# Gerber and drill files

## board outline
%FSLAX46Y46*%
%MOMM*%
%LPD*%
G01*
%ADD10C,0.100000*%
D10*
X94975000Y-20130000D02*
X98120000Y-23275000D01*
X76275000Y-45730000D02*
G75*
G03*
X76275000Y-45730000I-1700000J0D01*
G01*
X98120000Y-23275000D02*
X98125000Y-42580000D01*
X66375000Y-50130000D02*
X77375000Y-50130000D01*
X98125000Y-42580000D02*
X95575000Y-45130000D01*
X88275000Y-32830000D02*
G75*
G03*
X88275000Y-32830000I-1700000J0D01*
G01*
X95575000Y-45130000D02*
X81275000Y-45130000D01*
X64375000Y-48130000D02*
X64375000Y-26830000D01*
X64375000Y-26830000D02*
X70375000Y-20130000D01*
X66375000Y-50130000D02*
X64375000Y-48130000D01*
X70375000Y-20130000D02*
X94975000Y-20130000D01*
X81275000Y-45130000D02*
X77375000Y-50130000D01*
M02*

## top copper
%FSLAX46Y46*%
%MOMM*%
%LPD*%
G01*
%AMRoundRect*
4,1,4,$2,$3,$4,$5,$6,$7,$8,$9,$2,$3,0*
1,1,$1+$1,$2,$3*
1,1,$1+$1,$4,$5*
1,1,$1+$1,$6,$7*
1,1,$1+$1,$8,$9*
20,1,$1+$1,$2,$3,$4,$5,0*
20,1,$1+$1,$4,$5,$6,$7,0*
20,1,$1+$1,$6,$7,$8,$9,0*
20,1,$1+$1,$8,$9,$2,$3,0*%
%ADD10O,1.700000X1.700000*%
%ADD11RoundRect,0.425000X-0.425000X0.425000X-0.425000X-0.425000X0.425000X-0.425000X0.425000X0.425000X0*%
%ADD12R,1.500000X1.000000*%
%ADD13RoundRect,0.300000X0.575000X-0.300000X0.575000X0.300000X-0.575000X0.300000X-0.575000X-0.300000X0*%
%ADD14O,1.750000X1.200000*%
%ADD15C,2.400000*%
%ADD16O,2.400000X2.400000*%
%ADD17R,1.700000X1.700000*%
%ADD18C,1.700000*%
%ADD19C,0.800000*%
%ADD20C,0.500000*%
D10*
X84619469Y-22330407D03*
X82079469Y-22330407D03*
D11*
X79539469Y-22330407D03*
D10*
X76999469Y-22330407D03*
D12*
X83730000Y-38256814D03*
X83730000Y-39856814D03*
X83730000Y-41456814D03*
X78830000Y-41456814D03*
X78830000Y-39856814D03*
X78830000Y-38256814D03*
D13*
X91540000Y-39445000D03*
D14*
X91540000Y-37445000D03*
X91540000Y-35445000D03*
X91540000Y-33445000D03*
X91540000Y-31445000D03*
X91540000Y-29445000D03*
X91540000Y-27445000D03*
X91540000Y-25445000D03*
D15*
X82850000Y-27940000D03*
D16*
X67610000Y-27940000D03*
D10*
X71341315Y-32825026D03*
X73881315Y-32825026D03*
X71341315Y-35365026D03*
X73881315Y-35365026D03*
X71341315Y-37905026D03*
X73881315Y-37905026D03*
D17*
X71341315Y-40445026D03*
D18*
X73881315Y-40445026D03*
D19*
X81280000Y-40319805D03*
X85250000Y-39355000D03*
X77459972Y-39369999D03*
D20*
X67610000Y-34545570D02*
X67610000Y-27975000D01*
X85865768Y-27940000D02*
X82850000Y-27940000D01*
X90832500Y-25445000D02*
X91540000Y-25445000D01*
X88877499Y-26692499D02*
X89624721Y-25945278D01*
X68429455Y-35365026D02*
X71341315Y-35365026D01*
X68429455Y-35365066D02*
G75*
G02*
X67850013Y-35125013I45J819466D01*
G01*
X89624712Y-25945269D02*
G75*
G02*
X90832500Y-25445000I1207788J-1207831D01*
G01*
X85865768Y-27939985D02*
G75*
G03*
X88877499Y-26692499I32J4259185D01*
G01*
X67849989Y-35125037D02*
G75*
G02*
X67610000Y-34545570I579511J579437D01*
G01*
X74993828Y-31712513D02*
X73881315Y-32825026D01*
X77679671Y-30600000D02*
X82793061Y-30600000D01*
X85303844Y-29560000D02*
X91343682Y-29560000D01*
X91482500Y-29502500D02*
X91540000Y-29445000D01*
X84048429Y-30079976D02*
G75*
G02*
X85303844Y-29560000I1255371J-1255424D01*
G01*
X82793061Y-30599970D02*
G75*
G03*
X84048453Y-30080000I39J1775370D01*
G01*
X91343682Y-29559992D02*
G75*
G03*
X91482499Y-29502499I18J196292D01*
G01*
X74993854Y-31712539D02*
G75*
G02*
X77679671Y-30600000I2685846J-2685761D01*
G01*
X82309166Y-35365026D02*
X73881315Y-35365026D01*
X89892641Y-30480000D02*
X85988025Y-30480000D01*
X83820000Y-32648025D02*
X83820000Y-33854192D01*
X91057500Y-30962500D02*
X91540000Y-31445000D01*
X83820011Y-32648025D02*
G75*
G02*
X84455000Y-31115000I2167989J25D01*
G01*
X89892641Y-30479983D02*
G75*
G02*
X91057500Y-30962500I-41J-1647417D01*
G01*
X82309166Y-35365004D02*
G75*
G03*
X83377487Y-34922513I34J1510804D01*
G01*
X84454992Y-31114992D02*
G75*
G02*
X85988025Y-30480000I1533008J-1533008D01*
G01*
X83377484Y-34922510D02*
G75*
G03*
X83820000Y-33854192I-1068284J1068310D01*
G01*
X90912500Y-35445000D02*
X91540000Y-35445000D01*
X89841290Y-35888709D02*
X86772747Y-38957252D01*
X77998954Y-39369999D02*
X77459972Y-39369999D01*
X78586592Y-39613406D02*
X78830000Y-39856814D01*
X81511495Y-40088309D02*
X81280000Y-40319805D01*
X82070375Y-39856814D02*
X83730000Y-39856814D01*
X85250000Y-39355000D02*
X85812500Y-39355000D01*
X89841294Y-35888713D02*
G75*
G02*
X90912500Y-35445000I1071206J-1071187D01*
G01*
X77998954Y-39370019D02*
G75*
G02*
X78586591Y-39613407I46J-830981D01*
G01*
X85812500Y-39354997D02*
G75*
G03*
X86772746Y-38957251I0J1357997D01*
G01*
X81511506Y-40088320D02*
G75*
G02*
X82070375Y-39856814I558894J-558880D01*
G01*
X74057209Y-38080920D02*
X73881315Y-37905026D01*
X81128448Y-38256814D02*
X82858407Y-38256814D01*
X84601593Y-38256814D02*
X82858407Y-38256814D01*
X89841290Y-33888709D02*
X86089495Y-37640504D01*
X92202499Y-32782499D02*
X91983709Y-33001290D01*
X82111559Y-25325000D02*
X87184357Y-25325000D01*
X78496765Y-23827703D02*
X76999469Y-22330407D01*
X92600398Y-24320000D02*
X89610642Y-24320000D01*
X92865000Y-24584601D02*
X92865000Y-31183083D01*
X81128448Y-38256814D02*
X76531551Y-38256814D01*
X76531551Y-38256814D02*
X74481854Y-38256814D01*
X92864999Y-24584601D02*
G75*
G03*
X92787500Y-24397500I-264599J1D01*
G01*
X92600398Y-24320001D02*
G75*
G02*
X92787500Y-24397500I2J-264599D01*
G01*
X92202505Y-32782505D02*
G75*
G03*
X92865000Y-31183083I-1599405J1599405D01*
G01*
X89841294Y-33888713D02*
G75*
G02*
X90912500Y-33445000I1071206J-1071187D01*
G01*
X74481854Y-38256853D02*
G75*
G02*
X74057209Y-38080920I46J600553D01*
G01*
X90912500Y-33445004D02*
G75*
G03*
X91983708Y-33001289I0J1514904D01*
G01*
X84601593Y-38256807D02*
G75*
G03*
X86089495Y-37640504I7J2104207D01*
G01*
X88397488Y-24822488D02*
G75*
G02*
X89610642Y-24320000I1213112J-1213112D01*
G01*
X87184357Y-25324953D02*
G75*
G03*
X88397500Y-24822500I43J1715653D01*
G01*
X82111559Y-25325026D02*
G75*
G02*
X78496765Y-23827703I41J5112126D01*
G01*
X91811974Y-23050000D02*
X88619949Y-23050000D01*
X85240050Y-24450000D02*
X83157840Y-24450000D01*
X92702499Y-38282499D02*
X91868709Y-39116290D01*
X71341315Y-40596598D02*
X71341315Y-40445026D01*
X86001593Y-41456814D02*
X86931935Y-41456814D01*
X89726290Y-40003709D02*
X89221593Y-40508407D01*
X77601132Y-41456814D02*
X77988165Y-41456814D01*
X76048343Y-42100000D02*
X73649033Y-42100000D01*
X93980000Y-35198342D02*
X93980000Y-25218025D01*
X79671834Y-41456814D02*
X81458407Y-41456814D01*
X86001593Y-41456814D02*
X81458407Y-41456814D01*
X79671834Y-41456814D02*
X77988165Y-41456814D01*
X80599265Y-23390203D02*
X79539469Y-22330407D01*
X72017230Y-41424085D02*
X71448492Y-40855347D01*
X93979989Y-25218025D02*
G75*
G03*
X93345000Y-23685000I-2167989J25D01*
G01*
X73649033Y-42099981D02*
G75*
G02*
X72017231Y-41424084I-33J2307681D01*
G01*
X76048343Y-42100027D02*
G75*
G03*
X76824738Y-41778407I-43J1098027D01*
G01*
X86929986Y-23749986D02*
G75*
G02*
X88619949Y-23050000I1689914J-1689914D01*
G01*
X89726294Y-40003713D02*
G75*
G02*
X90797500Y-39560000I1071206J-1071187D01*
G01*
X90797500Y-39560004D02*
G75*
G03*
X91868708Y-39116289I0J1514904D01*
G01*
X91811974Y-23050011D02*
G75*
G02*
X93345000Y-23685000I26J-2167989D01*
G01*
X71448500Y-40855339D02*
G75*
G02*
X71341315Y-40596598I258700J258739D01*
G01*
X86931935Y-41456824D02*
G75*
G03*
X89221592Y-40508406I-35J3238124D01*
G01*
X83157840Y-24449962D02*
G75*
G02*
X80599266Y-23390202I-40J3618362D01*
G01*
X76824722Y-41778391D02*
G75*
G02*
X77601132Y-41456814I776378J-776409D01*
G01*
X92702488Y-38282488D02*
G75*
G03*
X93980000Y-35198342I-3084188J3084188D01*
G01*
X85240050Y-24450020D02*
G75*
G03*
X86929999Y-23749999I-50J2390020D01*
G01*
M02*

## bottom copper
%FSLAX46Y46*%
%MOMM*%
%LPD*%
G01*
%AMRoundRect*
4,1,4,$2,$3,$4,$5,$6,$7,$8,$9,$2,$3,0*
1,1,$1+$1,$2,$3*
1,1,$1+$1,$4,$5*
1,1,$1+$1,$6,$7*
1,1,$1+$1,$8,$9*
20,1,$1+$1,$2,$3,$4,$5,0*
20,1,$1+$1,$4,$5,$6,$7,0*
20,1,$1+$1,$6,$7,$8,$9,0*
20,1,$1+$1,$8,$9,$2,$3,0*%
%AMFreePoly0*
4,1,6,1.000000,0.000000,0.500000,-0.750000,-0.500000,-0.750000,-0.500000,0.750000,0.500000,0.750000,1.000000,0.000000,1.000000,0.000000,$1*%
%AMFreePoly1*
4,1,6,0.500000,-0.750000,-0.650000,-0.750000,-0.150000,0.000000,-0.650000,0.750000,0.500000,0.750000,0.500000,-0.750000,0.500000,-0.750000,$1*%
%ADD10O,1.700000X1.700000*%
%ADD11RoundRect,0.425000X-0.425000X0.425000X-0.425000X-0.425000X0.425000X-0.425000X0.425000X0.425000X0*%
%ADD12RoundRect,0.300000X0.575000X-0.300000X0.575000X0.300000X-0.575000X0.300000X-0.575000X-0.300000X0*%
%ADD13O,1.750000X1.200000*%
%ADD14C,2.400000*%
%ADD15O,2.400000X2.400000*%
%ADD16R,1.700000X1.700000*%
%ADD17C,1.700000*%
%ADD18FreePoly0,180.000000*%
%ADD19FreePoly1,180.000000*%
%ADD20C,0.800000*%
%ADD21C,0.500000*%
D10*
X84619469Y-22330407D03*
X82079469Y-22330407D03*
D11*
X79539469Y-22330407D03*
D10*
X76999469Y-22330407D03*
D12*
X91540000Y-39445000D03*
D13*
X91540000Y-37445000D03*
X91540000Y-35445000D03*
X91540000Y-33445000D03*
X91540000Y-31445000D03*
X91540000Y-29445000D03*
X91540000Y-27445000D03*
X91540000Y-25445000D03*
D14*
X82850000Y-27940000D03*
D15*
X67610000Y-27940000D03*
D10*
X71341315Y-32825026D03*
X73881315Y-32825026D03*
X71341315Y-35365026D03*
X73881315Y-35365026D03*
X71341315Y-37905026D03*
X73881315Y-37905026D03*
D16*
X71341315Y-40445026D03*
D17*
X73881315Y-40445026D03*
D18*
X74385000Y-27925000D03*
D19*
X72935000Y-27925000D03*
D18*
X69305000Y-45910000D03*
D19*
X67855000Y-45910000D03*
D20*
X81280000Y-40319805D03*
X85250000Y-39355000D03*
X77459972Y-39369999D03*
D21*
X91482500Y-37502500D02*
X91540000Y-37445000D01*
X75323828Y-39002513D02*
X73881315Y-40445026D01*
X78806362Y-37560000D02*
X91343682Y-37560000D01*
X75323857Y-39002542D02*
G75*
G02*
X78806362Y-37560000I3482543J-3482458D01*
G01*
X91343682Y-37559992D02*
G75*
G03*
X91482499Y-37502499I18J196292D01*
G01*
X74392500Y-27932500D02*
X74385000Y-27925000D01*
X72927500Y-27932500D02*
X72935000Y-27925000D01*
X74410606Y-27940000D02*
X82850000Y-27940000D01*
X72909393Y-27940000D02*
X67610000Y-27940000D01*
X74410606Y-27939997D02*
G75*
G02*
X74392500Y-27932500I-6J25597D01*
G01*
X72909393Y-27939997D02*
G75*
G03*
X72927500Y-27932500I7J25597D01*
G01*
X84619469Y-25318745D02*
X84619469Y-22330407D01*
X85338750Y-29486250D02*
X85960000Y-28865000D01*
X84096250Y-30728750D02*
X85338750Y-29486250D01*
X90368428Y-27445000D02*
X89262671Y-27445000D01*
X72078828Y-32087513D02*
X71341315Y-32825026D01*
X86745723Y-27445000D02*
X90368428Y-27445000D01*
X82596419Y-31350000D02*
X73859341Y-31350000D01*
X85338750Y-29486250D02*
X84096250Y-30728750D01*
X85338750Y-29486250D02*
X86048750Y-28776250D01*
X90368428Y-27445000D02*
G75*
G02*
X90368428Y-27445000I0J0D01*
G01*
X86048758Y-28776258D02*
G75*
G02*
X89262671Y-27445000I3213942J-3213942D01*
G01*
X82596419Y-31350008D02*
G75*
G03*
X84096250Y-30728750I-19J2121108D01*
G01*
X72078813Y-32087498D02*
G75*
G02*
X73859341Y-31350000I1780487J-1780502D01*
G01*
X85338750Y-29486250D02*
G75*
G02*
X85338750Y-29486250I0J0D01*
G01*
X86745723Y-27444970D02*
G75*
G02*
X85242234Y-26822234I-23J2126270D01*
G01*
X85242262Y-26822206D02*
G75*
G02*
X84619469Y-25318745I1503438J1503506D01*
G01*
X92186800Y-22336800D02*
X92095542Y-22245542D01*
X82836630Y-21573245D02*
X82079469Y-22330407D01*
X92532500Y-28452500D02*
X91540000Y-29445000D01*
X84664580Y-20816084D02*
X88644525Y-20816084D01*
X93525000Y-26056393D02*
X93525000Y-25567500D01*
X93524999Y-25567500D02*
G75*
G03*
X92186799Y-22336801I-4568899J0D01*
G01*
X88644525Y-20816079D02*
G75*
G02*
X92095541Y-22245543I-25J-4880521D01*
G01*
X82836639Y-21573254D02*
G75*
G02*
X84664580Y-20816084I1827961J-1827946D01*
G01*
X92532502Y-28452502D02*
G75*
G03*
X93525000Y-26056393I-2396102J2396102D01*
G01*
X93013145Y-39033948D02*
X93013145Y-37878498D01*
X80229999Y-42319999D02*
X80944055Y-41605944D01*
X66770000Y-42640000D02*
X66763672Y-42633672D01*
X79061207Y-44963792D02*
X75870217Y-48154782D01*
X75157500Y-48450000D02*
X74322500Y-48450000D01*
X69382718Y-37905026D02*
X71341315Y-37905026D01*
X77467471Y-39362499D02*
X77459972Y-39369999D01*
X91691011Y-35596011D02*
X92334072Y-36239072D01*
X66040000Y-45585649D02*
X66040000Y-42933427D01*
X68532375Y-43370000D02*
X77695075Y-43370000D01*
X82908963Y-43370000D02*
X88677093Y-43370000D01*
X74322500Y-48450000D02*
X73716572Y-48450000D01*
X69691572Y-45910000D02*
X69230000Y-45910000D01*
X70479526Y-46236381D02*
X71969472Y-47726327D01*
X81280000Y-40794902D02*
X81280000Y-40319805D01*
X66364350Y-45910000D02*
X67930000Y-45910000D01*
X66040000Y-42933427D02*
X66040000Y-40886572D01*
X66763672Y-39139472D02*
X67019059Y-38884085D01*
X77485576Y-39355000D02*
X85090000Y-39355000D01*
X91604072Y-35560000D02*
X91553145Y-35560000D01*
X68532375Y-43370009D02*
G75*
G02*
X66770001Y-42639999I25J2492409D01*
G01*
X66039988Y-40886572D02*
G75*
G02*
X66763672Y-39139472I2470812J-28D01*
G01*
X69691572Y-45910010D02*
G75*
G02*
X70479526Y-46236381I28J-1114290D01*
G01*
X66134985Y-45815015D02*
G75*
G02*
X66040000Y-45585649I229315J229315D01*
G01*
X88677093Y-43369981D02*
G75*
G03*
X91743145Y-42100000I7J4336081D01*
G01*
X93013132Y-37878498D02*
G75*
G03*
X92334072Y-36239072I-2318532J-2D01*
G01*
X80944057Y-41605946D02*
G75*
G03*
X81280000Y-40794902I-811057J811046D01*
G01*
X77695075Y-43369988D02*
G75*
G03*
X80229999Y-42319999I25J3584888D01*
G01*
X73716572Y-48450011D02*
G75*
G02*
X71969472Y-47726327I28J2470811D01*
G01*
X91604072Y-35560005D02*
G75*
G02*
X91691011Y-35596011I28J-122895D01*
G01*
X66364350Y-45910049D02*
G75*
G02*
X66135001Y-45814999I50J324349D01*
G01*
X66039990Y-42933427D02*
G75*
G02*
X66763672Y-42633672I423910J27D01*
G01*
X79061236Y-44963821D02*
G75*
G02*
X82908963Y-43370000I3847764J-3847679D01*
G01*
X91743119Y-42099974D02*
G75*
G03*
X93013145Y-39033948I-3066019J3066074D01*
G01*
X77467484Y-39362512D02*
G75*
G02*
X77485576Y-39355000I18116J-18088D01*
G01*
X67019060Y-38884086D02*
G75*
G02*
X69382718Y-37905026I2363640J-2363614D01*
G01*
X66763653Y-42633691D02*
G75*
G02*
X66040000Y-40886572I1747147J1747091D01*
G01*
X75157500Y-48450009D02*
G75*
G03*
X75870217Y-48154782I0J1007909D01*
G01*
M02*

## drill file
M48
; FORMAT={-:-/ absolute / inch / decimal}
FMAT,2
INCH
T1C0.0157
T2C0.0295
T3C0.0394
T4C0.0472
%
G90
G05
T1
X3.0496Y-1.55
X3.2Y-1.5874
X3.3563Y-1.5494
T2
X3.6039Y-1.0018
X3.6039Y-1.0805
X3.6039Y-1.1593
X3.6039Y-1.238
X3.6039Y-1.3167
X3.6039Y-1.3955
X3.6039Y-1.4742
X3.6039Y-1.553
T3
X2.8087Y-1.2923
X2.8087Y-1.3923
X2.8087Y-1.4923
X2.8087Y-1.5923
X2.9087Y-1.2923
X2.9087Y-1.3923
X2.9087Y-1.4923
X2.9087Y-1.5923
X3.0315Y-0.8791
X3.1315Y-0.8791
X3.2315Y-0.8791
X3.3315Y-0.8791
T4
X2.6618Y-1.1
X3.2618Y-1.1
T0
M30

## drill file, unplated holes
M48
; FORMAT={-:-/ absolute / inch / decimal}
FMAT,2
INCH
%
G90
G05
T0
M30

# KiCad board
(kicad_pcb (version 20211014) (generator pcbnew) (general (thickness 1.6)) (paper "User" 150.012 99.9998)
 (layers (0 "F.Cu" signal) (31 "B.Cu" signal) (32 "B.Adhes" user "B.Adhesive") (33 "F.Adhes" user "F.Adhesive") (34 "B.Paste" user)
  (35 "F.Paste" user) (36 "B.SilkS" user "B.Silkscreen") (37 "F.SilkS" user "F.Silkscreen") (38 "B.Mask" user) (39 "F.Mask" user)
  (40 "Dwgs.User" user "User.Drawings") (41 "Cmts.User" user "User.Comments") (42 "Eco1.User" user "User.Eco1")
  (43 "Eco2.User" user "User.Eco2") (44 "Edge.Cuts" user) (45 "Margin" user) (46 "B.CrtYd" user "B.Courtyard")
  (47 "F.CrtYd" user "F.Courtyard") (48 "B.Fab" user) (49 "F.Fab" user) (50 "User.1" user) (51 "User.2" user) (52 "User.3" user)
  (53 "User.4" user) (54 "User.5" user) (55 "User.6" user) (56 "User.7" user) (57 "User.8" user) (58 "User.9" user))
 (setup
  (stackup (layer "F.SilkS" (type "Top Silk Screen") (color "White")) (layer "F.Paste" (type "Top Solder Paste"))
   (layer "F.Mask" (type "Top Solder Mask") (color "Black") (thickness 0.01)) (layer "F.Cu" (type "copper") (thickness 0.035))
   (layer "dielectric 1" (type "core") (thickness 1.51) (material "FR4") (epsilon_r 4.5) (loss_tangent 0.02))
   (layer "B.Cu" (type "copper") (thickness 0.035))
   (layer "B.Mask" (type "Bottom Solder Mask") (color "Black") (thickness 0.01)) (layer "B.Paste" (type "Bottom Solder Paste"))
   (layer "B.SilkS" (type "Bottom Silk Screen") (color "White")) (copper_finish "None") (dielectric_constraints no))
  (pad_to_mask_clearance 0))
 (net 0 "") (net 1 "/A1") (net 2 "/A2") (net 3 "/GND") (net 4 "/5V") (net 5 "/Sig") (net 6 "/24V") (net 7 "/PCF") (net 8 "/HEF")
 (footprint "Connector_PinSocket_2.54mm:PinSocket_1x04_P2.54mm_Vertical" (layer "F.Cu") (at 84.619469 22.330407 -90)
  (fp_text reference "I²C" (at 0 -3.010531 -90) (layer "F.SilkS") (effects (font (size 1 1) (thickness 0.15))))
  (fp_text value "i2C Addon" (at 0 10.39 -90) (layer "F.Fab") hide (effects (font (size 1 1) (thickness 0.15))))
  (pad "1" thru_hole oval (at 0 0 270) (size 1.7 1.7) (drill 1) (layers *.Cu *.Mask) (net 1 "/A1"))
  (pad "2" thru_hole oval (at 0 2.54 270) (size 1.7 1.7) (drill 1) (layers *.Cu *.Mask) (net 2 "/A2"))
  (pad "3" thru_hole roundrect (at 0 5.08 270) (size 1.7 1.7) (drill 1) (layers *.Cu *.Mask) (roundrect_rratio 0.25) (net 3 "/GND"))
  (pad "4" thru_hole oval (at 0 7.62 270) (size 1.7 1.7) (drill 1) (layers *.Cu *.Mask) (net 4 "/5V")))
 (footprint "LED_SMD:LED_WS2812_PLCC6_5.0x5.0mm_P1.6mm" (layer "F.Cu") (at 81.28 39.856814)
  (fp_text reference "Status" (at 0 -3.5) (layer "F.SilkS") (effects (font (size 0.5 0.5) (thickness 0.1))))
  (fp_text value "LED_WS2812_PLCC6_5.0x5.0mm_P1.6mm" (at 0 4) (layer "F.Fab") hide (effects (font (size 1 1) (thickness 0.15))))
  (pad "1" smd rect (at 2.45 -1.6) (size 1.5 1) (layers "F.Cu" "F.Paste" "F.Mask") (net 4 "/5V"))
  (pad "2" smd rect (at 2.45 0) (size 1.5 1) (layers "F.Cu" "F.Paste" "F.Mask") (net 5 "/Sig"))
  (pad "3" smd rect (at 2.45 1.6) (size 1.5 1) (layers "F.Cu" "F.Paste" "F.Mask") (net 3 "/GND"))
  (pad "4" smd rect (at -2.45 1.6) (size 1.5 1) (layers "F.Cu" "F.Paste" "F.Mask") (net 3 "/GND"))
  (pad "5" smd rect (at -2.45 0) (size 1.5 1) (layers "F.Cu" "F.Paste" "F.Mask") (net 5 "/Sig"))
  (pad "6" smd rect (at -2.45 -1.6) (size 1.5 1) (layers "F.Cu" "F.Paste" "F.Mask") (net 4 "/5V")))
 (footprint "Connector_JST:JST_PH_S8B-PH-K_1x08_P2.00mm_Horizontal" (layer "F.Cu") (at 91.54 39.445 90)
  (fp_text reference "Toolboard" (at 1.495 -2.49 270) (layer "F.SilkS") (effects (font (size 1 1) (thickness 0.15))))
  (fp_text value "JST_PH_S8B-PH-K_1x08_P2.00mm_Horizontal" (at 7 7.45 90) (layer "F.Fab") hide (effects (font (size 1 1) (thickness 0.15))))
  (pad "1" thru_hole roundrect (at 0 0 90) (size 1.2 1.75) (drill 0.75) (layers *.Cu *.Mask) (roundrect_rratio 0.25) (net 3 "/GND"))
  (pad "2" thru_hole oval (at 2 0 90) (size 1.2 1.75) (drill 0.75) (layers *.Cu *.Mask) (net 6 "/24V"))
  (pad "3" thru_hole oval (at 4 0 90) (size 1.2 1.75) (drill 0.75) (layers *.Cu *.Mask) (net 5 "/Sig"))
  (pad "4" thru_hole oval (at 6 0 90) (size 1.2 1.75) (drill 0.75) (layers *.Cu *.Mask) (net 4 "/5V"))
  (pad "5" thru_hole oval (at 8 0 90) (size 1.2 1.75) (drill 0.75) (layers *.Cu *.Mask) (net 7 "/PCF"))
  (pad "6" thru_hole oval (at 10 0 90) (size 1.2 1.75) (drill 0.75) (layers *.Cu *.Mask) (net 2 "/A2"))
  (pad "7" thru_hole oval (at 12 0 90) (size 1.2 1.75) (drill 0.75) (layers *.Cu *.Mask) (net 1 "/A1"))
  (pad "8" thru_hole oval (at 14 0 90) (size 1.2 1.75) (drill 0.75) (layers *.Cu *.Mask) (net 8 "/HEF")))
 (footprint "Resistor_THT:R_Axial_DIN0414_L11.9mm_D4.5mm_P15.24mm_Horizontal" (layer "F.Cu") (at 82.85 27.94 180)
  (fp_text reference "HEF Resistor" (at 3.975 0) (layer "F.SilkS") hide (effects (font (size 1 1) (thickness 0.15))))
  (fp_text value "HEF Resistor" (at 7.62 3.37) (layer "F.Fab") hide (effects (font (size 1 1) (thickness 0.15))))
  (pad "1" thru_hole circle (at 0 0 180) (size 2.4 2.4) (drill 1.2) (layers *.Cu *.Mask) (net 8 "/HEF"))
  (pad "2" thru_hole oval (at 15.24 0 180) (size 2.4 2.4) (drill 1.2) (layers *.Cu *.Mask) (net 8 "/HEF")))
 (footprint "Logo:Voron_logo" (layer "F.Cu") (at 80.775 32.73)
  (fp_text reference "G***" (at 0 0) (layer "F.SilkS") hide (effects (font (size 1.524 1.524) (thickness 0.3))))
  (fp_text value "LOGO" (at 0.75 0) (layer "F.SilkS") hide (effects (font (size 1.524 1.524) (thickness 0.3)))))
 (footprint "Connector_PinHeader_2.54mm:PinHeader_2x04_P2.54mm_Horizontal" (layer "F.Cu") (at 63.261315 32.825026)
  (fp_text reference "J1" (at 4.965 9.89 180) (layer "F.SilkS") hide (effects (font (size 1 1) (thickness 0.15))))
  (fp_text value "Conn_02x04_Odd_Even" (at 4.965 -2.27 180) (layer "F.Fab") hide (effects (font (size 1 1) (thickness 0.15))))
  (pad "1" thru_hole oval (at 8.08 0 180) (size 1.7 1.7) (drill 1) (layers *.Cu *.Mask) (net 1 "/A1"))
  (pad "2" thru_hole oval (at 10.62 0 180) (size 1.7 1.7) (drill 1) (layers *.Cu *.Mask) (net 2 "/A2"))
  (pad "3" thru_hole oval (at 8.08 2.54 180) (size 1.7 1.7) (drill 1) (layers *.Cu *.Mask) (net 8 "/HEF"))
  (pad "4" thru_hole oval (at 10.62 2.54 180) (size 1.7 1.7) (drill 1) (layers *.Cu *.Mask) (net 7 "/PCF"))
  (pad "5" thru_hole oval (at 8.08 5.08 180) (size 1.7 1.7) (drill 1) (layers *.Cu *.Mask) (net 5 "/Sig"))
  (pad "6" thru_hole oval (at 10.62 5.08 180) (size 1.7 1.7) (drill 1) (layers *.Cu *.Mask) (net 4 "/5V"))
  (pad "7" thru_hole rect (at 8.08 7.62 180) (size 1.7 1.7) (drill 1) (layers *.Cu *.Mask) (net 3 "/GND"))
  (pad "8" thru_hole circle (at 10.62 7.62 180) (size 1.7 1.7) (drill 1) (layers *.Cu *.Mask) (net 6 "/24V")))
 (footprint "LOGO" (layer "F.Cu") (at 93.98 21.59)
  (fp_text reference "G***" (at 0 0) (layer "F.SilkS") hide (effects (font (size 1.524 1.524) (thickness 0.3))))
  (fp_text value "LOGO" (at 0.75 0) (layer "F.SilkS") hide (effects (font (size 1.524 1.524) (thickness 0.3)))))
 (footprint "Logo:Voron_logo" (layer "B.Cu") (at 80.775 32.73 180)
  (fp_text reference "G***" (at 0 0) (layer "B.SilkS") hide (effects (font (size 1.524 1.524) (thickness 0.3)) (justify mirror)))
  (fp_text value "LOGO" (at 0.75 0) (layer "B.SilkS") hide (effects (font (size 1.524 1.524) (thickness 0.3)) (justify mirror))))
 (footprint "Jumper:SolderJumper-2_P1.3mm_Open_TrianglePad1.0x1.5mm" (layer "B.Cu") (at 73.66 27.925 180)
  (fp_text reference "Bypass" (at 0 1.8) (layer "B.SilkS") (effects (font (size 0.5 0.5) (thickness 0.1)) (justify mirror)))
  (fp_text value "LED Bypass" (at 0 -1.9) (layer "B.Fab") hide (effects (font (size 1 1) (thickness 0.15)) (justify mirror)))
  (pad "1" smd custom (at -0.725 0 180) (size 0.3 0.3) (layers "B.Cu" "B.Mask") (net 8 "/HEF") (zone_connect 2)
   (options (clearance outline) (anchor rect)) (primitives))
  (pad "2" smd custom (at 0.725 0 180) (size 0.3 0.3) (layers "B.Cu" "B.Mask") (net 8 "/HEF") (zone_connect 2)
   (options (clearance outline) (anchor rect)) (primitives)))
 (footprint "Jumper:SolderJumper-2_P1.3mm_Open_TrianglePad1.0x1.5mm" (layer "B.Cu") (at 68.58 45.91 180)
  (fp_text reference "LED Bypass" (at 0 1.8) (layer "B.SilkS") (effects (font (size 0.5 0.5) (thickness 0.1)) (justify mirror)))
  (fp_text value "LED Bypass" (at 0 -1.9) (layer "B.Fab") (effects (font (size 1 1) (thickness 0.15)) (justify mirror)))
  (pad "1" smd custom (at -0.725 0 180) (size 0.3 0.3) (layers "B.Cu" "B.Mask") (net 5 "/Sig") (zone_connect 2)
   (options (clearance outline) (anchor rect)) (primitives))
  (pad "2" smd custom (at 0.725 0 180) (size 0.3 0.3) (layers "B.Cu" "B.Mask") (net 5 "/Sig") (zone_connect 2)
   (options (clearance outline) (anchor rect)) (primitives)))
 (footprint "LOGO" (layer "B.Cu") (at 71.12 22.86 180)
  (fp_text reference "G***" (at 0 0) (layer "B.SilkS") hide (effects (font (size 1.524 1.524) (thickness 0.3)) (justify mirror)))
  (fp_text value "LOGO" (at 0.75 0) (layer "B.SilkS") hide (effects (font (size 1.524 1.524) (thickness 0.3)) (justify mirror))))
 (gr_line (start 94.975 20.13) (end 98.12 23.275) (layer "Edge.Cuts") (width 0.1))
 (gr_circle (center 74.575 45.73) (end 76.275 45.73) (layer "Edge.Cuts") (width 0.1) (fill none))
 (gr_line (start 98.12 23.275) (end 98.125 42.58) (layer "Edge.Cuts") (width 0.1))
 (gr_line (start 66.375 50.13) (end 77.375 50.13) (layer "Edge.Cuts") (width 0.1))
 (gr_line (start 98.125 42.58) (end 95.575 45.13) (layer "Edge.Cuts") (width 0.1))
 (gr_circle (center 86.575 32.83) (end 88.275 32.83) (layer "Edge.Cuts") (width 0.1) (fill none))
 (gr_line (start 95.575 45.13) (end 81.275 45.13) (layer "Edge.Cuts") (width 0.1))
 (gr_line (start 64.375 48.13) (end 64.375 26.83) (layer "Edge.Cuts") (width 0.1))
 (gr_line (start 64.375 26.83) (end 70.375 20.13) (layer "Edge.Cuts") (width 0.1))
 (gr_line (start 66.375 50.13) (end 64.375 48.13) (layer "Edge.Cuts") (width 0.1))
 (gr_line (start 70.375 20.13) (end 94.975 20.13) (layer "Edge.Cuts") (width 0.1))
 (gr_line (start 81.275 45.13) (end 77.375 50.13) (layer "Edge.Cuts") (width 0.1))
 (segment (start 91.4825 37.5025) (end 91.54 37.445) (width 0.5) (layer "B.Cu") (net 6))
 (segment (start 75.323828 39.002513) (end 73.881315 40.445026) (width 0.5) (layer "B.Cu") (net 6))
 (segment (start 78.806362 37.56) (end 91.343682 37.56) (width 0.5) (layer "B.Cu") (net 6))
 (arc (start 78.806362 37.56) (mid 76.921628 37.934896) (end 75.323828 39.002513) (width 0.5) (layer "B.Cu") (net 6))
 (arc (start 91.4825 37.5025) (mid 91.418809 37.545056) (end 91.343682 37.56) (width 0.5) (layer "B.Cu") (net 6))
 (segment (start 67.61 34.54557) (end 67.61 27.975) (width 0.5) (layer "F.Cu") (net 8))
 (segment (start 85.865768 27.94) (end 82.85 27.94) (width 0.5) (layer "F.Cu") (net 8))
 (segment (start 90.8325 25.445) (end 91.54 25.445) (width 0.5) (layer "F.Cu") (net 8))
 (segment (start 88.877499 26.692499) (end 89.624721 25.945278) (width 0.5) (layer "F.Cu") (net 8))
 (segment (start 68.429455 35.365026) (end 71.341315 35.365026) (width 0.5) (layer "F.Cu") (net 8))
 (arc (start 67.850013 35.125013) (mid 68.115863 35.302648) (end 68.429455 35.365026) (width 0.5) (layer "F.Cu") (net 8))
 (arc (start 90.8325 25.445) (mid 90.178854 25.575018) (end 89.624721 25.945278) (width 0.5) (layer "F.Cu") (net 8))
 (arc (start 88.877499 26.692499) (mid 87.495705 27.615785) (end 85.865768 27.94) (width 0.5) (layer "F.Cu") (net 8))
 (arc (start 67.61 34.54557) (mid 67.672377 34.859162) (end 67.850013 35.125013) (width 0.5) (layer "F.Cu") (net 8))
 (segment (start 74.3925 27.9325) (end 74.385 27.925) (width 0.5) (layer "B.Cu") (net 8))
 (segment (start 72.9275 27.9325) (end 72.935 27.925) (width 0.5) (layer "B.Cu") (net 8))
 (segment (start 74.410606 27.94) (end 82.85 27.94) (width 0.5) (layer "B.Cu") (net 8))
 (segment (start 72.909393 27.94) (end 67.61 27.94) (width 0.5) (layer "B.Cu") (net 8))
 (arc (start 74.3925 27.9325) (mid 74.400807 27.93805) (end 74.410606 27.94) (width 0.5) (layer "B.Cu") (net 8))
 (arc (start 72.9275 27.9325) (mid 72.919192 27.93805) (end 72.909393 27.94) (width 0.5) (layer "B.Cu") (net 8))
 (segment (start 84.619469 25.318745) (end 84.619469 22.330407) (width 0.5) (layer "B.Cu") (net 1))
 (segment (start 85.33875 29.48625) (end 85.96 28.865) (width 0.5) (layer "B.Cu") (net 1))
 (segment (start 84.09625 30.72875) (end 85.33875 29.48625) (width 0.5) (layer "B.Cu") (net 1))
 (segment (start 90.368428 27.445) (end 89.262671 27.445) (width 0.5) (layer "B.Cu") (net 1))
 (segment (start 72.078828 32.087513) (end 71.341315 32.825026) (width 0.5) (layer "B.Cu") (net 1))
 (segment (start 86.745723 27.445) (end 90.368428 27.445) (width 0.5) (layer "B.Cu") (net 1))
 (segment (start 82.596419 31.35) (end 73.859341 31.35) (width 0.5) (layer "B.Cu") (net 1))
 (segment (start 85.33875 29.48625) (end 84.09625 30.72875) (width 0.5) (layer "B.Cu") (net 1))
 (segment (start 85.33875 29.48625) (end 86.04875 28.77625) (width 0.5) (layer "B.Cu") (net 1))
 (arc (start 90.368428 27.445) (mid 90.368428 27.445) (end 90.368428 27.445) (width 0.5) (layer "B.Cu") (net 1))
 (arc (start 89.262671 27.445) (mid 87.523309 27.79098) (end 86.04875 28.77625) (width 0.5) (layer "B.Cu") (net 1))
 (arc (start 84.09625 30.72875) (mid 83.408121 31.188542) (end 82.596419 31.35) (width 0.5) (layer "B.Cu") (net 1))
 (arc (start 73.859341 31.35) (mid 72.895734 31.541673) (end 72.078828 32.087513) (width 0.5) (layer "B.Cu") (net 1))
 (arc (start 85.33875 29.48625) (mid 85.33875 29.48625) (end 85.33875 29.48625) (width 0.5) (layer "B.Cu") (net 1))
 (arc (start 85.242234 26.822234) (mid 85.93204 27.283148) (end 86.745723 27.445) (width 0.5) (layer "B.Cu") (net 1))
 (arc (start 84.619469 25.318745) (mid 84.78132 26.132427) (end 85.242234 26.822234) (width 0.5) (layer "B.Cu") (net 1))
 (segment (start 74.993828 31.712513) (end 73.881315 32.825026) (width 0.5) (layer "F.Cu") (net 2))
 (segment (start 77.679671 30.6) (end 82.793061 30.6) (width 0.5) (layer "F.Cu") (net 2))
 (segment (start 85.303844 29.56) (end 91.343682 29.56) (width 0.5) (layer "F.Cu") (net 2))
 (segment (start 91.4825 29.5025) (end 91.54 29.445) (width 0.5) (layer "F.Cu") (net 2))
 (arc (start 85.303844 29.56) (mid 84.624431 29.695143) (end 84.048453 30.08) (width 0.5) (layer "F.Cu") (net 2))
 (arc (start 84.048453 30.08) (mid 83.472474 30.464856) (end 82.793061 30.6) (width 0.5) (layer "F.Cu") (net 2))
 (arc (start 91.4825 29.5025) (mid 91.418809 29.545056) (end 91.343682 29.56) (width 0.5) (layer "F.Cu") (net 2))
 (arc (start 77.679671 30.6) (mid 76.226103 30.889132) (end 74.993828 31.712513) (width 0.5) (layer "F.Cu") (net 2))
 (segment (start 92.1868 22.3368) (end 92.095542 22.245542) (width 0.5) (layer "B.Cu") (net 2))
 (segment (start 82.83663 21.573245) (end 82.079469 22.330407) (width 0.5) (layer "B.Cu") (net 2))
 (segment (start 92.5325 28.4525) (end 91.54 29.445) (width 0.5) (layer "B.Cu") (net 2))
 (segment (start 84.66458 20.816084) (end 88.644525 20.816084) (width 0.5) (layer "B.Cu") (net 2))
 (segment (start 93.525 26.056393) (end 93.525 25.5675) (width 0.5) (layer "B.Cu") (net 2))
 (arc (start 92.1868 22.3368) (mid 93.177213 23.819057) (end 93.525 25.5675) (width 0.5) (layer "B.Cu") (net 2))
 (arc (start 92.095542 22.245542) (mid 90.512201 21.187588) (end 88.644525 20.816084) (width 0.5) (layer "B.Cu") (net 2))
 (arc (start 84.66458 20.816084) (mid 83.6753 21.012863) (end 82.83663 21.573245) (width 0.5) (layer "B.Cu") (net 2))
 (arc (start 93.525 26.056393) (mid 93.267057 27.353156) (end 92.5325 28.4525) (width 0.5) (layer "B.Cu") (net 2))
 (segment (start 82.309166 35.365026) (end 73.881315 35.365026) (width 0.5) (layer "F.Cu") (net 7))
 (segment (start 89.892641 30.48) (end 85.988025 30.48) (width 0.5) (layer "F.Cu") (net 7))
 (segment (start 83.82 32.648025) (end 83.82 33.854192) (width 0.5) (layer "F.Cu") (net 7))
 (segment (start 91.0575 30.9625) (end 91.54 31.445) (width 0.5) (layer "F.Cu") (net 7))
 (arc (start 84.455 31.115) (mid 83.985031 31.818357) (end 83.82 32.648025) (width 0.5) (layer "F.Cu") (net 7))
 (arc (start 91.0575 30.9625) (mid 90.523058 30.605397) (end 89.892641 30.48) (width 0.5) (layer "F.Cu") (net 7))
 (arc (start 83.377487 34.922513) (mid 82.887337 35.25002) (end 82.309166 35.365026) (width 0.5) (layer "F.Cu") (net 7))
 (arc (start 85.988025 30.48) (mid 85.158357 30.645031) (end 84.455 31.115) (width 0.5) (layer "F.Cu") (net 7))
 (arc (start 83.82 33.854192) (mid 83.704994 34.432363) (end 83.377487 34.922513) (width 0.5) (layer "F.Cu") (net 7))
 (segment (start 90.9125 35.445) (end 91.54 35.445) (width 0.5) (layer "F.Cu") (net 5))
 (segment (start 89.84129 35.888709) (end 86.772747 38.957252) (width 0.5) (layer "F.Cu") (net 5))
 (segment (start 77.998954 39.369999) (end 77.459972 39.369999) (width 0.5) (layer "F.Cu") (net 5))
 (segment (start 78.586592 39.613406) (end 78.83 39.856814) (width 0.5) (layer "F.Cu") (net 5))
 (segment (start 81.511495 40.088309) (end 81.28 40.319805) (width 0.5) (layer "F.Cu") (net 5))
 (segment (start 82.070375 39.856814) (end 83.73 39.856814) (width 0.5) (layer "F.Cu") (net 5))
 (segment (start 85.25 39.355) (end 85.8125 39.355) (width 0.5) (layer "F.Cu") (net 5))
 (via blind (at 81.28 40.319805) (size 0.8) (drill 0.4) (layers "F.Cu" "B.Cu") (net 5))
 (via blind (at 85.25 39.355) (size 0.8) (drill 0.4) (layers "F.Cu" "B.Cu") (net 5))
 (via blind (at 77.459972 39.369999) (size 0.8) (drill 0.4) (layers "F.Cu" "B.Cu") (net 5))
 (arc (start 90.9125 35.445) (mid 90.332765 35.560316) (end 89.84129 35.888709) (width 0.5) (layer "F.Cu") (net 5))
 (arc (start 78.586592 39.613406) (mid 78.316981 39.433258) (end 77.998954 39.369999) (width 0.5) (layer "F.Cu") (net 5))
 (arc (start 86.772747 38.957252) (mid 86.332182 39.251628) (end 85.8125 39.355) (width 0.5) (layer "F.Cu") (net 5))
 (arc (start 82.070375 39.856814) (mid 81.767911 39.916977) (end 81.511495 40.088309) (width 0.5) (layer "F.Cu") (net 5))
 (segment (start 93.013145 39.033948) (end 93.013145 37.878498) (width 0.5) (layer "B.Cu") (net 5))
 (segment (start 80.229999 42.319999) (end 80.944055 41.605944) (width 0.5) (layer "B.Cu") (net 5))
 (segment (start 66.77 42.64) (end 66.763672 42.633672) (width 0.5) (layer "B.Cu") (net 5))
 (segment (start 79.061207 44.963792) (end 75.870217 48.154782) (width 0.5) (layer "B.Cu") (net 5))
 (segment (start 75.1575 48.45) (end 74.3225 48.45) (width 0.5) (layer "B.Cu") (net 5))
 (segment (start 69.382718 37.905026) (end 71.341315 37.905026) (width 0.5) (layer "B.Cu") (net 5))
 (segment (start 77.467471 39.362499) (end 77.459972 39.369999) (width 0.5) (layer "B.Cu") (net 5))
 (segment (start 91.691011 35.596011) (end 92.334072 36.239072) (width 0.5) (layer "B.Cu") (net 5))
 (segment (start 66.04 45.585649) (end 66.04 42.933427) (width 0.5) (layer "B.Cu") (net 5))
 (segment (start 68.532375 43.37) (end 77.695075 43.37) (width 0.5) (layer "B.Cu") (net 5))
 (segment (start 82.908963 43.37) (end 88.677093 43.37) (width 0.5) (layer "B.Cu") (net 5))
 (segment (start 74.3225 48.45) (end 73.716572 48.45) (width 0.5) (layer "B.Cu") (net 5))
 (segment (start 69.691572 45.91) (end 69.23 45.91) (width 0.5) (layer "B.Cu") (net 5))
 (segment (start 70.479526 46.236381) (end 71.969472 47.726327) (width 0.5) (layer "B.Cu") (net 5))
 (segment (start 81.28 40.794902) (end 81.28 40.319805) (width 0.5) (layer "B.Cu") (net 5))
 (segment (start 66.36435 45.91) (end 67.93 45.91) (width 0.5) (layer "B.Cu") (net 5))
 (segment (start 66.04 42.933427) (end 66.04 40.886572) (width 0.5) (layer "B.Cu") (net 5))
 (segment (start 66.763672 39.139472) (end 67.019059 38.884085) (width 0.5) (layer "B.Cu") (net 5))
 (segment (start 77.485576 39.355) (end 85.09 39.355) (width 0.5) (layer "B.Cu") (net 5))
 (segment (start 91.604072 35.56) (end 91.553145 35.56) (width 0.5) (layer "B.Cu") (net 5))
 (arc (start 66.77 42.64) (mid 67.578584 43.180279) (end 68.532375 43.37) (width 0.5) (layer "B.Cu") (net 5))
 (arc (start 66.763672 39.139472) (mid 66.228076 39.941048) (end 66.04 40.886572) (width 0.5) (layer "B.Cu") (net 5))
 (arc (start 70.479526 46.236381) (mid 70.118009 45.994823) (end 69.691572 45.91) (width 0.5) (layer "B.Cu") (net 5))
 (arc (start 66.04 45.585649) (mid 66.064689 45.709773) (end 66.135 45.815) (width 0.5) (layer "B.Cu") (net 5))
 (arc (start 91.743145 42.1) (mid 90.336428 43.039937) (end 88.677093 43.37) (width 0.5) (layer "B.Cu") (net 5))
 (arc (start 92.334072 36.239072) (mid 92.836659 36.991247) (end 93.013145 37.878498) (width 0.5) (layer "B.Cu") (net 5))
 (arc (start 81.28 40.794902) (mid 81.19269 41.233835) (end 80.944055 41.605944) (width 0.5) (layer "B.Cu") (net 5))
 (arc (start 80.229999 42.319999) (mid 79.066966 43.097113) (end 77.695075 43.37) (width 0.5) (layer "B.Cu") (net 5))
 (arc (start 71.969472 47.726327) (mid 72.771048 48.261923) (end 73.716572 48.45) (width 0.5) (layer "B.Cu") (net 5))
 (arc (start 91.691011 35.596011) (mid 91.651123 35.569358) (end 91.604072 35.56) (width 0.5) (layer "B.Cu") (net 5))
 (arc (start 66.135 45.815) (mid 66.240226 45.88531) (end 66.36435 45.91) (width 0.5) (layer "B.Cu") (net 5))
 (arc (start 66.763672 42.633672) (mid 66.301691 42.541778) (end 66.04 42.933427) (width 0.5) (layer "B.Cu") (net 5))
 (arc (start 82.908963 43.37) (mid 80.826572 43.784213) (end 79.061207 44.963792) (width 0.5) (layer "B.Cu") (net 5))
 (arc (start 93.013145 39.033948) (mid 92.683082 40.693283) (end 91.743145 42.1) (width 0.5) (layer "B.Cu") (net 5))
 (arc (start 77.485576 39.355) (mid 77.475777 39.356948) (end 77.467471 39.362499) (width 0.5) (layer "B.Cu") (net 5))
 (arc (start 69.382718 37.905026) (mid 68.103515 38.159475) (end 67.019059 38.884085) (width 0.5) (layer "B.Cu") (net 5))
 (arc (start 66.04 40.886572) (mid 66.228076 41.832095) (end 66.763672 42.633672) (width 0.5) (layer "B.Cu") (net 5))
 (arc (start 75.870217 48.154782) (mid 75.543219 48.373275) (end 75.1575 48.45) (width 0.5) (layer "B.Cu") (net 5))
 (segment (start 74.057209 38.08092) (end 73.881315 37.905026) (width 0.5) (layer "F.Cu") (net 4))
 (segment (start 81.128448 38.256814) (end 82.858407 38.256814) (width 0.5) (layer "F.Cu") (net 4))
 (segment (start 84.601593 38.256814) (end 82.858407 38.256814) (width 0.5) (layer "F.Cu") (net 4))
 (segment (start 89.84129 33.888709) (end 86.089495 37.640504) (width 0.5) (layer "F.Cu") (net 4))
 (segment (start 92.202499 32.782499) (end 91.983709 33.00129) (width 0.5) (layer "F.Cu") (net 4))
 (segment (start 82.111559 25.325) (end 87.184357 25.325) (width 0.5) (layer "F.Cu") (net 4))
 (segment (start 78.496765 23.827703) (end 76.999469 22.330407) (width 0.5) (layer "F.Cu") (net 4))
 (segment (start 92.600398 24.32) (end 89.610642 24.32) (width 0.5) (layer "F.Cu") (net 4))
 (segment (start 92.865 24.584601) (end 92.865 31.183083) (width 0.5) (layer "F.Cu") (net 4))
 (segment (start 81.128448 38.256814) (end 76.531551 38.256814) (width 0.5) (layer "F.Cu") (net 4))
 (segment (start 76.531551 38.256814) (end 74.481854 38.256814) (width 0.5) (layer "F.Cu") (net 4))
 (arc (start 92.7875 24.3975) (mid 92.844858 24.483342) (end 92.865 24.584601) (width 0.5) (layer "F.Cu") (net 4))
 (arc (start 92.7875 24.3975) (mid 92.701656 24.340141) (end 92.600398 24.32) (width 0.5) (layer "F.Cu") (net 4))
 (arc (start 92.865 31.183083) (mid 92.692821 32.048681) (end 92.202499 32.782499) (width 0.5) (layer "F.Cu") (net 4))
 (arc (start 90.9125 33.445) (mid 90.332765 33.560316) (end 89.84129 33.888709) (width 0.5) (layer "F.Cu") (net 4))
 (arc (start 74.057209 38.08092) (mid 74.252037 38.2111) (end 74.481854 38.256814) (width 0.5) (layer "F.Cu") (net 4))
 (arc (start 91.983709 33.00129) (mid 91.492234 33.329683) (end 90.9125 33.445) (width 0.5) (layer "F.Cu") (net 4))
 (arc (start 86.089495 37.640504) (mid 85.406839 38.09664) (end 84.601593 38.256814) (width 0.5) (layer "F.Cu") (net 4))
 (arc (start 89.610642 24.32) (mid 88.954094 24.450595) (end 88.3975 24.8225) (width 0.5) (layer "F.Cu") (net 4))
 (arc (start 88.3975 24.8225) (mid 87.840905 25.194404) (end 87.184357 25.325) (width 0.5) (layer "F.Cu") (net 4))
 (arc (start 78.496765 23.827703) (mid 80.155246 24.935865) (end 82.111559 25.325) (width 0.5) (layer "F.Cu") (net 4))
 (segment (start 91.811974 23.05) (end 88.619949 23.05) (width 0.5) (layer "F.Cu") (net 3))
 (segment (start 85.24005 24.45) (end 83.15784 24.45) (width 0.5) (layer "F.Cu") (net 3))
 (segment (start 92.702499 38.282499) (end 91.868709 39.11629) (width 0.5) (layer "F.Cu") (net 3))
 (segment (start 71.341315 40.596598) (end 71.341315 40.445026) (width 0.5) (layer "F.Cu") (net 3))
 (segment (start 86.001593 41.456814) (end 86.931935 41.456814) (width 0.5) (layer "F.Cu") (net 3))
 (segment (start 89.72629 40.003709) (end 89.221593 40.508407) (width 0.5) (layer "F.Cu") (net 3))
 (segment (start 77.601132 41.456814) (end 77.988165 41.456814) (width 0.5) (layer "F.Cu") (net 3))
 (segment (start 76.048343 42.1) (end 73.649033 42.1) (width 0.5) (layer "F.Cu") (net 3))
 (segment (start 93.98 35.198342) (end 93.98 25.218025) (width 0.5) (layer "F.Cu") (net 3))
 (segment (start 79.671834 41.456814) (end 81.458407 41.456814) (width 0.5) (layer "F.Cu") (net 3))
 (segment (start 86.001593 41.456814) (end 81.458407 41.456814) (width 0.5) (layer "F.Cu") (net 3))
 (segment (start 79.671834 41.456814) (end 77.988165 41.456814) (width 0.5) (layer "F.Cu") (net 3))
 (segment (start 80.599265 23.390203) (end 79.539469 22.330407) (width 0.5) (layer "F.Cu") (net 3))
 (segment (start 72.01723 41.424085) (end 71.448492 40.855347) (width 0.5) (layer "F.Cu") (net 3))
 (arc (start 93.345 23.685) (mid 93.814968 24.388357) (end 93.98 25.218025) (width 0.5) (layer "F.Cu") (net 3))
 (arc (start 72.01723 41.424085) (mid 72.765907 41.924335) (end 73.649033 42.1) (width 0.5) (layer "F.Cu") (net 3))
 (arc (start 76.824738 41.778407) (mid 76.468525 42.01642) (end 76.048343 42.1) (width 0.5) (layer "F.Cu") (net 3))
 (arc (start 88.619949 23.05) (mid 87.705355 23.231924) (end 86.93 23.75) (width 0.5) (layer "F.Cu") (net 3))
 (arc (start 90.7975 39.56) (mid 90.217765 39.675316) (end 89.72629 40.003709) (width 0.5) (layer "F.Cu") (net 3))
 (arc (start 91.868709 39.11629) (mid 91.377234 39.444683) (end 90.7975 39.56) (width 0.5) (layer "F.Cu") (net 3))
 (arc (start 93.345 23.685) (mid 92.641641 23.215031) (end 91.811974 23.05) (width 0.5) (layer "F.Cu") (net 3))
 (arc (start 71.341315 40.596598) (mid 71.369169 40.736632) (end 71.448492 40.855347) (width 0.5) (layer "F.Cu") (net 3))
 (arc (start 89.221593 40.508407) (mid 88.171089 41.210331) (end 86.931935 41.456814) (width 0.5) (layer "F.Cu") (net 3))
 (arc (start 80.599265 23.390203) (mid 81.773149 24.174567) (end 83.15784 24.45) (width 0.5) (layer "F.Cu") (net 3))
 (arc (start 77.601132 41.456814) (mid 77.18095 41.540393) (end 76.824738 41.778407) (width 0.5) (layer "F.Cu") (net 3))
 (arc (start 93.98 35.198342) (mid 93.647988 36.867476) (end 92.702499 38.282499) (width 0.5) (layer "F.Cu") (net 3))
 (arc (start 86.93 23.75) (mid 86.154644 24.268075) (end 85.24005 24.45) (width 0.5) (layer "F.Cu") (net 3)))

